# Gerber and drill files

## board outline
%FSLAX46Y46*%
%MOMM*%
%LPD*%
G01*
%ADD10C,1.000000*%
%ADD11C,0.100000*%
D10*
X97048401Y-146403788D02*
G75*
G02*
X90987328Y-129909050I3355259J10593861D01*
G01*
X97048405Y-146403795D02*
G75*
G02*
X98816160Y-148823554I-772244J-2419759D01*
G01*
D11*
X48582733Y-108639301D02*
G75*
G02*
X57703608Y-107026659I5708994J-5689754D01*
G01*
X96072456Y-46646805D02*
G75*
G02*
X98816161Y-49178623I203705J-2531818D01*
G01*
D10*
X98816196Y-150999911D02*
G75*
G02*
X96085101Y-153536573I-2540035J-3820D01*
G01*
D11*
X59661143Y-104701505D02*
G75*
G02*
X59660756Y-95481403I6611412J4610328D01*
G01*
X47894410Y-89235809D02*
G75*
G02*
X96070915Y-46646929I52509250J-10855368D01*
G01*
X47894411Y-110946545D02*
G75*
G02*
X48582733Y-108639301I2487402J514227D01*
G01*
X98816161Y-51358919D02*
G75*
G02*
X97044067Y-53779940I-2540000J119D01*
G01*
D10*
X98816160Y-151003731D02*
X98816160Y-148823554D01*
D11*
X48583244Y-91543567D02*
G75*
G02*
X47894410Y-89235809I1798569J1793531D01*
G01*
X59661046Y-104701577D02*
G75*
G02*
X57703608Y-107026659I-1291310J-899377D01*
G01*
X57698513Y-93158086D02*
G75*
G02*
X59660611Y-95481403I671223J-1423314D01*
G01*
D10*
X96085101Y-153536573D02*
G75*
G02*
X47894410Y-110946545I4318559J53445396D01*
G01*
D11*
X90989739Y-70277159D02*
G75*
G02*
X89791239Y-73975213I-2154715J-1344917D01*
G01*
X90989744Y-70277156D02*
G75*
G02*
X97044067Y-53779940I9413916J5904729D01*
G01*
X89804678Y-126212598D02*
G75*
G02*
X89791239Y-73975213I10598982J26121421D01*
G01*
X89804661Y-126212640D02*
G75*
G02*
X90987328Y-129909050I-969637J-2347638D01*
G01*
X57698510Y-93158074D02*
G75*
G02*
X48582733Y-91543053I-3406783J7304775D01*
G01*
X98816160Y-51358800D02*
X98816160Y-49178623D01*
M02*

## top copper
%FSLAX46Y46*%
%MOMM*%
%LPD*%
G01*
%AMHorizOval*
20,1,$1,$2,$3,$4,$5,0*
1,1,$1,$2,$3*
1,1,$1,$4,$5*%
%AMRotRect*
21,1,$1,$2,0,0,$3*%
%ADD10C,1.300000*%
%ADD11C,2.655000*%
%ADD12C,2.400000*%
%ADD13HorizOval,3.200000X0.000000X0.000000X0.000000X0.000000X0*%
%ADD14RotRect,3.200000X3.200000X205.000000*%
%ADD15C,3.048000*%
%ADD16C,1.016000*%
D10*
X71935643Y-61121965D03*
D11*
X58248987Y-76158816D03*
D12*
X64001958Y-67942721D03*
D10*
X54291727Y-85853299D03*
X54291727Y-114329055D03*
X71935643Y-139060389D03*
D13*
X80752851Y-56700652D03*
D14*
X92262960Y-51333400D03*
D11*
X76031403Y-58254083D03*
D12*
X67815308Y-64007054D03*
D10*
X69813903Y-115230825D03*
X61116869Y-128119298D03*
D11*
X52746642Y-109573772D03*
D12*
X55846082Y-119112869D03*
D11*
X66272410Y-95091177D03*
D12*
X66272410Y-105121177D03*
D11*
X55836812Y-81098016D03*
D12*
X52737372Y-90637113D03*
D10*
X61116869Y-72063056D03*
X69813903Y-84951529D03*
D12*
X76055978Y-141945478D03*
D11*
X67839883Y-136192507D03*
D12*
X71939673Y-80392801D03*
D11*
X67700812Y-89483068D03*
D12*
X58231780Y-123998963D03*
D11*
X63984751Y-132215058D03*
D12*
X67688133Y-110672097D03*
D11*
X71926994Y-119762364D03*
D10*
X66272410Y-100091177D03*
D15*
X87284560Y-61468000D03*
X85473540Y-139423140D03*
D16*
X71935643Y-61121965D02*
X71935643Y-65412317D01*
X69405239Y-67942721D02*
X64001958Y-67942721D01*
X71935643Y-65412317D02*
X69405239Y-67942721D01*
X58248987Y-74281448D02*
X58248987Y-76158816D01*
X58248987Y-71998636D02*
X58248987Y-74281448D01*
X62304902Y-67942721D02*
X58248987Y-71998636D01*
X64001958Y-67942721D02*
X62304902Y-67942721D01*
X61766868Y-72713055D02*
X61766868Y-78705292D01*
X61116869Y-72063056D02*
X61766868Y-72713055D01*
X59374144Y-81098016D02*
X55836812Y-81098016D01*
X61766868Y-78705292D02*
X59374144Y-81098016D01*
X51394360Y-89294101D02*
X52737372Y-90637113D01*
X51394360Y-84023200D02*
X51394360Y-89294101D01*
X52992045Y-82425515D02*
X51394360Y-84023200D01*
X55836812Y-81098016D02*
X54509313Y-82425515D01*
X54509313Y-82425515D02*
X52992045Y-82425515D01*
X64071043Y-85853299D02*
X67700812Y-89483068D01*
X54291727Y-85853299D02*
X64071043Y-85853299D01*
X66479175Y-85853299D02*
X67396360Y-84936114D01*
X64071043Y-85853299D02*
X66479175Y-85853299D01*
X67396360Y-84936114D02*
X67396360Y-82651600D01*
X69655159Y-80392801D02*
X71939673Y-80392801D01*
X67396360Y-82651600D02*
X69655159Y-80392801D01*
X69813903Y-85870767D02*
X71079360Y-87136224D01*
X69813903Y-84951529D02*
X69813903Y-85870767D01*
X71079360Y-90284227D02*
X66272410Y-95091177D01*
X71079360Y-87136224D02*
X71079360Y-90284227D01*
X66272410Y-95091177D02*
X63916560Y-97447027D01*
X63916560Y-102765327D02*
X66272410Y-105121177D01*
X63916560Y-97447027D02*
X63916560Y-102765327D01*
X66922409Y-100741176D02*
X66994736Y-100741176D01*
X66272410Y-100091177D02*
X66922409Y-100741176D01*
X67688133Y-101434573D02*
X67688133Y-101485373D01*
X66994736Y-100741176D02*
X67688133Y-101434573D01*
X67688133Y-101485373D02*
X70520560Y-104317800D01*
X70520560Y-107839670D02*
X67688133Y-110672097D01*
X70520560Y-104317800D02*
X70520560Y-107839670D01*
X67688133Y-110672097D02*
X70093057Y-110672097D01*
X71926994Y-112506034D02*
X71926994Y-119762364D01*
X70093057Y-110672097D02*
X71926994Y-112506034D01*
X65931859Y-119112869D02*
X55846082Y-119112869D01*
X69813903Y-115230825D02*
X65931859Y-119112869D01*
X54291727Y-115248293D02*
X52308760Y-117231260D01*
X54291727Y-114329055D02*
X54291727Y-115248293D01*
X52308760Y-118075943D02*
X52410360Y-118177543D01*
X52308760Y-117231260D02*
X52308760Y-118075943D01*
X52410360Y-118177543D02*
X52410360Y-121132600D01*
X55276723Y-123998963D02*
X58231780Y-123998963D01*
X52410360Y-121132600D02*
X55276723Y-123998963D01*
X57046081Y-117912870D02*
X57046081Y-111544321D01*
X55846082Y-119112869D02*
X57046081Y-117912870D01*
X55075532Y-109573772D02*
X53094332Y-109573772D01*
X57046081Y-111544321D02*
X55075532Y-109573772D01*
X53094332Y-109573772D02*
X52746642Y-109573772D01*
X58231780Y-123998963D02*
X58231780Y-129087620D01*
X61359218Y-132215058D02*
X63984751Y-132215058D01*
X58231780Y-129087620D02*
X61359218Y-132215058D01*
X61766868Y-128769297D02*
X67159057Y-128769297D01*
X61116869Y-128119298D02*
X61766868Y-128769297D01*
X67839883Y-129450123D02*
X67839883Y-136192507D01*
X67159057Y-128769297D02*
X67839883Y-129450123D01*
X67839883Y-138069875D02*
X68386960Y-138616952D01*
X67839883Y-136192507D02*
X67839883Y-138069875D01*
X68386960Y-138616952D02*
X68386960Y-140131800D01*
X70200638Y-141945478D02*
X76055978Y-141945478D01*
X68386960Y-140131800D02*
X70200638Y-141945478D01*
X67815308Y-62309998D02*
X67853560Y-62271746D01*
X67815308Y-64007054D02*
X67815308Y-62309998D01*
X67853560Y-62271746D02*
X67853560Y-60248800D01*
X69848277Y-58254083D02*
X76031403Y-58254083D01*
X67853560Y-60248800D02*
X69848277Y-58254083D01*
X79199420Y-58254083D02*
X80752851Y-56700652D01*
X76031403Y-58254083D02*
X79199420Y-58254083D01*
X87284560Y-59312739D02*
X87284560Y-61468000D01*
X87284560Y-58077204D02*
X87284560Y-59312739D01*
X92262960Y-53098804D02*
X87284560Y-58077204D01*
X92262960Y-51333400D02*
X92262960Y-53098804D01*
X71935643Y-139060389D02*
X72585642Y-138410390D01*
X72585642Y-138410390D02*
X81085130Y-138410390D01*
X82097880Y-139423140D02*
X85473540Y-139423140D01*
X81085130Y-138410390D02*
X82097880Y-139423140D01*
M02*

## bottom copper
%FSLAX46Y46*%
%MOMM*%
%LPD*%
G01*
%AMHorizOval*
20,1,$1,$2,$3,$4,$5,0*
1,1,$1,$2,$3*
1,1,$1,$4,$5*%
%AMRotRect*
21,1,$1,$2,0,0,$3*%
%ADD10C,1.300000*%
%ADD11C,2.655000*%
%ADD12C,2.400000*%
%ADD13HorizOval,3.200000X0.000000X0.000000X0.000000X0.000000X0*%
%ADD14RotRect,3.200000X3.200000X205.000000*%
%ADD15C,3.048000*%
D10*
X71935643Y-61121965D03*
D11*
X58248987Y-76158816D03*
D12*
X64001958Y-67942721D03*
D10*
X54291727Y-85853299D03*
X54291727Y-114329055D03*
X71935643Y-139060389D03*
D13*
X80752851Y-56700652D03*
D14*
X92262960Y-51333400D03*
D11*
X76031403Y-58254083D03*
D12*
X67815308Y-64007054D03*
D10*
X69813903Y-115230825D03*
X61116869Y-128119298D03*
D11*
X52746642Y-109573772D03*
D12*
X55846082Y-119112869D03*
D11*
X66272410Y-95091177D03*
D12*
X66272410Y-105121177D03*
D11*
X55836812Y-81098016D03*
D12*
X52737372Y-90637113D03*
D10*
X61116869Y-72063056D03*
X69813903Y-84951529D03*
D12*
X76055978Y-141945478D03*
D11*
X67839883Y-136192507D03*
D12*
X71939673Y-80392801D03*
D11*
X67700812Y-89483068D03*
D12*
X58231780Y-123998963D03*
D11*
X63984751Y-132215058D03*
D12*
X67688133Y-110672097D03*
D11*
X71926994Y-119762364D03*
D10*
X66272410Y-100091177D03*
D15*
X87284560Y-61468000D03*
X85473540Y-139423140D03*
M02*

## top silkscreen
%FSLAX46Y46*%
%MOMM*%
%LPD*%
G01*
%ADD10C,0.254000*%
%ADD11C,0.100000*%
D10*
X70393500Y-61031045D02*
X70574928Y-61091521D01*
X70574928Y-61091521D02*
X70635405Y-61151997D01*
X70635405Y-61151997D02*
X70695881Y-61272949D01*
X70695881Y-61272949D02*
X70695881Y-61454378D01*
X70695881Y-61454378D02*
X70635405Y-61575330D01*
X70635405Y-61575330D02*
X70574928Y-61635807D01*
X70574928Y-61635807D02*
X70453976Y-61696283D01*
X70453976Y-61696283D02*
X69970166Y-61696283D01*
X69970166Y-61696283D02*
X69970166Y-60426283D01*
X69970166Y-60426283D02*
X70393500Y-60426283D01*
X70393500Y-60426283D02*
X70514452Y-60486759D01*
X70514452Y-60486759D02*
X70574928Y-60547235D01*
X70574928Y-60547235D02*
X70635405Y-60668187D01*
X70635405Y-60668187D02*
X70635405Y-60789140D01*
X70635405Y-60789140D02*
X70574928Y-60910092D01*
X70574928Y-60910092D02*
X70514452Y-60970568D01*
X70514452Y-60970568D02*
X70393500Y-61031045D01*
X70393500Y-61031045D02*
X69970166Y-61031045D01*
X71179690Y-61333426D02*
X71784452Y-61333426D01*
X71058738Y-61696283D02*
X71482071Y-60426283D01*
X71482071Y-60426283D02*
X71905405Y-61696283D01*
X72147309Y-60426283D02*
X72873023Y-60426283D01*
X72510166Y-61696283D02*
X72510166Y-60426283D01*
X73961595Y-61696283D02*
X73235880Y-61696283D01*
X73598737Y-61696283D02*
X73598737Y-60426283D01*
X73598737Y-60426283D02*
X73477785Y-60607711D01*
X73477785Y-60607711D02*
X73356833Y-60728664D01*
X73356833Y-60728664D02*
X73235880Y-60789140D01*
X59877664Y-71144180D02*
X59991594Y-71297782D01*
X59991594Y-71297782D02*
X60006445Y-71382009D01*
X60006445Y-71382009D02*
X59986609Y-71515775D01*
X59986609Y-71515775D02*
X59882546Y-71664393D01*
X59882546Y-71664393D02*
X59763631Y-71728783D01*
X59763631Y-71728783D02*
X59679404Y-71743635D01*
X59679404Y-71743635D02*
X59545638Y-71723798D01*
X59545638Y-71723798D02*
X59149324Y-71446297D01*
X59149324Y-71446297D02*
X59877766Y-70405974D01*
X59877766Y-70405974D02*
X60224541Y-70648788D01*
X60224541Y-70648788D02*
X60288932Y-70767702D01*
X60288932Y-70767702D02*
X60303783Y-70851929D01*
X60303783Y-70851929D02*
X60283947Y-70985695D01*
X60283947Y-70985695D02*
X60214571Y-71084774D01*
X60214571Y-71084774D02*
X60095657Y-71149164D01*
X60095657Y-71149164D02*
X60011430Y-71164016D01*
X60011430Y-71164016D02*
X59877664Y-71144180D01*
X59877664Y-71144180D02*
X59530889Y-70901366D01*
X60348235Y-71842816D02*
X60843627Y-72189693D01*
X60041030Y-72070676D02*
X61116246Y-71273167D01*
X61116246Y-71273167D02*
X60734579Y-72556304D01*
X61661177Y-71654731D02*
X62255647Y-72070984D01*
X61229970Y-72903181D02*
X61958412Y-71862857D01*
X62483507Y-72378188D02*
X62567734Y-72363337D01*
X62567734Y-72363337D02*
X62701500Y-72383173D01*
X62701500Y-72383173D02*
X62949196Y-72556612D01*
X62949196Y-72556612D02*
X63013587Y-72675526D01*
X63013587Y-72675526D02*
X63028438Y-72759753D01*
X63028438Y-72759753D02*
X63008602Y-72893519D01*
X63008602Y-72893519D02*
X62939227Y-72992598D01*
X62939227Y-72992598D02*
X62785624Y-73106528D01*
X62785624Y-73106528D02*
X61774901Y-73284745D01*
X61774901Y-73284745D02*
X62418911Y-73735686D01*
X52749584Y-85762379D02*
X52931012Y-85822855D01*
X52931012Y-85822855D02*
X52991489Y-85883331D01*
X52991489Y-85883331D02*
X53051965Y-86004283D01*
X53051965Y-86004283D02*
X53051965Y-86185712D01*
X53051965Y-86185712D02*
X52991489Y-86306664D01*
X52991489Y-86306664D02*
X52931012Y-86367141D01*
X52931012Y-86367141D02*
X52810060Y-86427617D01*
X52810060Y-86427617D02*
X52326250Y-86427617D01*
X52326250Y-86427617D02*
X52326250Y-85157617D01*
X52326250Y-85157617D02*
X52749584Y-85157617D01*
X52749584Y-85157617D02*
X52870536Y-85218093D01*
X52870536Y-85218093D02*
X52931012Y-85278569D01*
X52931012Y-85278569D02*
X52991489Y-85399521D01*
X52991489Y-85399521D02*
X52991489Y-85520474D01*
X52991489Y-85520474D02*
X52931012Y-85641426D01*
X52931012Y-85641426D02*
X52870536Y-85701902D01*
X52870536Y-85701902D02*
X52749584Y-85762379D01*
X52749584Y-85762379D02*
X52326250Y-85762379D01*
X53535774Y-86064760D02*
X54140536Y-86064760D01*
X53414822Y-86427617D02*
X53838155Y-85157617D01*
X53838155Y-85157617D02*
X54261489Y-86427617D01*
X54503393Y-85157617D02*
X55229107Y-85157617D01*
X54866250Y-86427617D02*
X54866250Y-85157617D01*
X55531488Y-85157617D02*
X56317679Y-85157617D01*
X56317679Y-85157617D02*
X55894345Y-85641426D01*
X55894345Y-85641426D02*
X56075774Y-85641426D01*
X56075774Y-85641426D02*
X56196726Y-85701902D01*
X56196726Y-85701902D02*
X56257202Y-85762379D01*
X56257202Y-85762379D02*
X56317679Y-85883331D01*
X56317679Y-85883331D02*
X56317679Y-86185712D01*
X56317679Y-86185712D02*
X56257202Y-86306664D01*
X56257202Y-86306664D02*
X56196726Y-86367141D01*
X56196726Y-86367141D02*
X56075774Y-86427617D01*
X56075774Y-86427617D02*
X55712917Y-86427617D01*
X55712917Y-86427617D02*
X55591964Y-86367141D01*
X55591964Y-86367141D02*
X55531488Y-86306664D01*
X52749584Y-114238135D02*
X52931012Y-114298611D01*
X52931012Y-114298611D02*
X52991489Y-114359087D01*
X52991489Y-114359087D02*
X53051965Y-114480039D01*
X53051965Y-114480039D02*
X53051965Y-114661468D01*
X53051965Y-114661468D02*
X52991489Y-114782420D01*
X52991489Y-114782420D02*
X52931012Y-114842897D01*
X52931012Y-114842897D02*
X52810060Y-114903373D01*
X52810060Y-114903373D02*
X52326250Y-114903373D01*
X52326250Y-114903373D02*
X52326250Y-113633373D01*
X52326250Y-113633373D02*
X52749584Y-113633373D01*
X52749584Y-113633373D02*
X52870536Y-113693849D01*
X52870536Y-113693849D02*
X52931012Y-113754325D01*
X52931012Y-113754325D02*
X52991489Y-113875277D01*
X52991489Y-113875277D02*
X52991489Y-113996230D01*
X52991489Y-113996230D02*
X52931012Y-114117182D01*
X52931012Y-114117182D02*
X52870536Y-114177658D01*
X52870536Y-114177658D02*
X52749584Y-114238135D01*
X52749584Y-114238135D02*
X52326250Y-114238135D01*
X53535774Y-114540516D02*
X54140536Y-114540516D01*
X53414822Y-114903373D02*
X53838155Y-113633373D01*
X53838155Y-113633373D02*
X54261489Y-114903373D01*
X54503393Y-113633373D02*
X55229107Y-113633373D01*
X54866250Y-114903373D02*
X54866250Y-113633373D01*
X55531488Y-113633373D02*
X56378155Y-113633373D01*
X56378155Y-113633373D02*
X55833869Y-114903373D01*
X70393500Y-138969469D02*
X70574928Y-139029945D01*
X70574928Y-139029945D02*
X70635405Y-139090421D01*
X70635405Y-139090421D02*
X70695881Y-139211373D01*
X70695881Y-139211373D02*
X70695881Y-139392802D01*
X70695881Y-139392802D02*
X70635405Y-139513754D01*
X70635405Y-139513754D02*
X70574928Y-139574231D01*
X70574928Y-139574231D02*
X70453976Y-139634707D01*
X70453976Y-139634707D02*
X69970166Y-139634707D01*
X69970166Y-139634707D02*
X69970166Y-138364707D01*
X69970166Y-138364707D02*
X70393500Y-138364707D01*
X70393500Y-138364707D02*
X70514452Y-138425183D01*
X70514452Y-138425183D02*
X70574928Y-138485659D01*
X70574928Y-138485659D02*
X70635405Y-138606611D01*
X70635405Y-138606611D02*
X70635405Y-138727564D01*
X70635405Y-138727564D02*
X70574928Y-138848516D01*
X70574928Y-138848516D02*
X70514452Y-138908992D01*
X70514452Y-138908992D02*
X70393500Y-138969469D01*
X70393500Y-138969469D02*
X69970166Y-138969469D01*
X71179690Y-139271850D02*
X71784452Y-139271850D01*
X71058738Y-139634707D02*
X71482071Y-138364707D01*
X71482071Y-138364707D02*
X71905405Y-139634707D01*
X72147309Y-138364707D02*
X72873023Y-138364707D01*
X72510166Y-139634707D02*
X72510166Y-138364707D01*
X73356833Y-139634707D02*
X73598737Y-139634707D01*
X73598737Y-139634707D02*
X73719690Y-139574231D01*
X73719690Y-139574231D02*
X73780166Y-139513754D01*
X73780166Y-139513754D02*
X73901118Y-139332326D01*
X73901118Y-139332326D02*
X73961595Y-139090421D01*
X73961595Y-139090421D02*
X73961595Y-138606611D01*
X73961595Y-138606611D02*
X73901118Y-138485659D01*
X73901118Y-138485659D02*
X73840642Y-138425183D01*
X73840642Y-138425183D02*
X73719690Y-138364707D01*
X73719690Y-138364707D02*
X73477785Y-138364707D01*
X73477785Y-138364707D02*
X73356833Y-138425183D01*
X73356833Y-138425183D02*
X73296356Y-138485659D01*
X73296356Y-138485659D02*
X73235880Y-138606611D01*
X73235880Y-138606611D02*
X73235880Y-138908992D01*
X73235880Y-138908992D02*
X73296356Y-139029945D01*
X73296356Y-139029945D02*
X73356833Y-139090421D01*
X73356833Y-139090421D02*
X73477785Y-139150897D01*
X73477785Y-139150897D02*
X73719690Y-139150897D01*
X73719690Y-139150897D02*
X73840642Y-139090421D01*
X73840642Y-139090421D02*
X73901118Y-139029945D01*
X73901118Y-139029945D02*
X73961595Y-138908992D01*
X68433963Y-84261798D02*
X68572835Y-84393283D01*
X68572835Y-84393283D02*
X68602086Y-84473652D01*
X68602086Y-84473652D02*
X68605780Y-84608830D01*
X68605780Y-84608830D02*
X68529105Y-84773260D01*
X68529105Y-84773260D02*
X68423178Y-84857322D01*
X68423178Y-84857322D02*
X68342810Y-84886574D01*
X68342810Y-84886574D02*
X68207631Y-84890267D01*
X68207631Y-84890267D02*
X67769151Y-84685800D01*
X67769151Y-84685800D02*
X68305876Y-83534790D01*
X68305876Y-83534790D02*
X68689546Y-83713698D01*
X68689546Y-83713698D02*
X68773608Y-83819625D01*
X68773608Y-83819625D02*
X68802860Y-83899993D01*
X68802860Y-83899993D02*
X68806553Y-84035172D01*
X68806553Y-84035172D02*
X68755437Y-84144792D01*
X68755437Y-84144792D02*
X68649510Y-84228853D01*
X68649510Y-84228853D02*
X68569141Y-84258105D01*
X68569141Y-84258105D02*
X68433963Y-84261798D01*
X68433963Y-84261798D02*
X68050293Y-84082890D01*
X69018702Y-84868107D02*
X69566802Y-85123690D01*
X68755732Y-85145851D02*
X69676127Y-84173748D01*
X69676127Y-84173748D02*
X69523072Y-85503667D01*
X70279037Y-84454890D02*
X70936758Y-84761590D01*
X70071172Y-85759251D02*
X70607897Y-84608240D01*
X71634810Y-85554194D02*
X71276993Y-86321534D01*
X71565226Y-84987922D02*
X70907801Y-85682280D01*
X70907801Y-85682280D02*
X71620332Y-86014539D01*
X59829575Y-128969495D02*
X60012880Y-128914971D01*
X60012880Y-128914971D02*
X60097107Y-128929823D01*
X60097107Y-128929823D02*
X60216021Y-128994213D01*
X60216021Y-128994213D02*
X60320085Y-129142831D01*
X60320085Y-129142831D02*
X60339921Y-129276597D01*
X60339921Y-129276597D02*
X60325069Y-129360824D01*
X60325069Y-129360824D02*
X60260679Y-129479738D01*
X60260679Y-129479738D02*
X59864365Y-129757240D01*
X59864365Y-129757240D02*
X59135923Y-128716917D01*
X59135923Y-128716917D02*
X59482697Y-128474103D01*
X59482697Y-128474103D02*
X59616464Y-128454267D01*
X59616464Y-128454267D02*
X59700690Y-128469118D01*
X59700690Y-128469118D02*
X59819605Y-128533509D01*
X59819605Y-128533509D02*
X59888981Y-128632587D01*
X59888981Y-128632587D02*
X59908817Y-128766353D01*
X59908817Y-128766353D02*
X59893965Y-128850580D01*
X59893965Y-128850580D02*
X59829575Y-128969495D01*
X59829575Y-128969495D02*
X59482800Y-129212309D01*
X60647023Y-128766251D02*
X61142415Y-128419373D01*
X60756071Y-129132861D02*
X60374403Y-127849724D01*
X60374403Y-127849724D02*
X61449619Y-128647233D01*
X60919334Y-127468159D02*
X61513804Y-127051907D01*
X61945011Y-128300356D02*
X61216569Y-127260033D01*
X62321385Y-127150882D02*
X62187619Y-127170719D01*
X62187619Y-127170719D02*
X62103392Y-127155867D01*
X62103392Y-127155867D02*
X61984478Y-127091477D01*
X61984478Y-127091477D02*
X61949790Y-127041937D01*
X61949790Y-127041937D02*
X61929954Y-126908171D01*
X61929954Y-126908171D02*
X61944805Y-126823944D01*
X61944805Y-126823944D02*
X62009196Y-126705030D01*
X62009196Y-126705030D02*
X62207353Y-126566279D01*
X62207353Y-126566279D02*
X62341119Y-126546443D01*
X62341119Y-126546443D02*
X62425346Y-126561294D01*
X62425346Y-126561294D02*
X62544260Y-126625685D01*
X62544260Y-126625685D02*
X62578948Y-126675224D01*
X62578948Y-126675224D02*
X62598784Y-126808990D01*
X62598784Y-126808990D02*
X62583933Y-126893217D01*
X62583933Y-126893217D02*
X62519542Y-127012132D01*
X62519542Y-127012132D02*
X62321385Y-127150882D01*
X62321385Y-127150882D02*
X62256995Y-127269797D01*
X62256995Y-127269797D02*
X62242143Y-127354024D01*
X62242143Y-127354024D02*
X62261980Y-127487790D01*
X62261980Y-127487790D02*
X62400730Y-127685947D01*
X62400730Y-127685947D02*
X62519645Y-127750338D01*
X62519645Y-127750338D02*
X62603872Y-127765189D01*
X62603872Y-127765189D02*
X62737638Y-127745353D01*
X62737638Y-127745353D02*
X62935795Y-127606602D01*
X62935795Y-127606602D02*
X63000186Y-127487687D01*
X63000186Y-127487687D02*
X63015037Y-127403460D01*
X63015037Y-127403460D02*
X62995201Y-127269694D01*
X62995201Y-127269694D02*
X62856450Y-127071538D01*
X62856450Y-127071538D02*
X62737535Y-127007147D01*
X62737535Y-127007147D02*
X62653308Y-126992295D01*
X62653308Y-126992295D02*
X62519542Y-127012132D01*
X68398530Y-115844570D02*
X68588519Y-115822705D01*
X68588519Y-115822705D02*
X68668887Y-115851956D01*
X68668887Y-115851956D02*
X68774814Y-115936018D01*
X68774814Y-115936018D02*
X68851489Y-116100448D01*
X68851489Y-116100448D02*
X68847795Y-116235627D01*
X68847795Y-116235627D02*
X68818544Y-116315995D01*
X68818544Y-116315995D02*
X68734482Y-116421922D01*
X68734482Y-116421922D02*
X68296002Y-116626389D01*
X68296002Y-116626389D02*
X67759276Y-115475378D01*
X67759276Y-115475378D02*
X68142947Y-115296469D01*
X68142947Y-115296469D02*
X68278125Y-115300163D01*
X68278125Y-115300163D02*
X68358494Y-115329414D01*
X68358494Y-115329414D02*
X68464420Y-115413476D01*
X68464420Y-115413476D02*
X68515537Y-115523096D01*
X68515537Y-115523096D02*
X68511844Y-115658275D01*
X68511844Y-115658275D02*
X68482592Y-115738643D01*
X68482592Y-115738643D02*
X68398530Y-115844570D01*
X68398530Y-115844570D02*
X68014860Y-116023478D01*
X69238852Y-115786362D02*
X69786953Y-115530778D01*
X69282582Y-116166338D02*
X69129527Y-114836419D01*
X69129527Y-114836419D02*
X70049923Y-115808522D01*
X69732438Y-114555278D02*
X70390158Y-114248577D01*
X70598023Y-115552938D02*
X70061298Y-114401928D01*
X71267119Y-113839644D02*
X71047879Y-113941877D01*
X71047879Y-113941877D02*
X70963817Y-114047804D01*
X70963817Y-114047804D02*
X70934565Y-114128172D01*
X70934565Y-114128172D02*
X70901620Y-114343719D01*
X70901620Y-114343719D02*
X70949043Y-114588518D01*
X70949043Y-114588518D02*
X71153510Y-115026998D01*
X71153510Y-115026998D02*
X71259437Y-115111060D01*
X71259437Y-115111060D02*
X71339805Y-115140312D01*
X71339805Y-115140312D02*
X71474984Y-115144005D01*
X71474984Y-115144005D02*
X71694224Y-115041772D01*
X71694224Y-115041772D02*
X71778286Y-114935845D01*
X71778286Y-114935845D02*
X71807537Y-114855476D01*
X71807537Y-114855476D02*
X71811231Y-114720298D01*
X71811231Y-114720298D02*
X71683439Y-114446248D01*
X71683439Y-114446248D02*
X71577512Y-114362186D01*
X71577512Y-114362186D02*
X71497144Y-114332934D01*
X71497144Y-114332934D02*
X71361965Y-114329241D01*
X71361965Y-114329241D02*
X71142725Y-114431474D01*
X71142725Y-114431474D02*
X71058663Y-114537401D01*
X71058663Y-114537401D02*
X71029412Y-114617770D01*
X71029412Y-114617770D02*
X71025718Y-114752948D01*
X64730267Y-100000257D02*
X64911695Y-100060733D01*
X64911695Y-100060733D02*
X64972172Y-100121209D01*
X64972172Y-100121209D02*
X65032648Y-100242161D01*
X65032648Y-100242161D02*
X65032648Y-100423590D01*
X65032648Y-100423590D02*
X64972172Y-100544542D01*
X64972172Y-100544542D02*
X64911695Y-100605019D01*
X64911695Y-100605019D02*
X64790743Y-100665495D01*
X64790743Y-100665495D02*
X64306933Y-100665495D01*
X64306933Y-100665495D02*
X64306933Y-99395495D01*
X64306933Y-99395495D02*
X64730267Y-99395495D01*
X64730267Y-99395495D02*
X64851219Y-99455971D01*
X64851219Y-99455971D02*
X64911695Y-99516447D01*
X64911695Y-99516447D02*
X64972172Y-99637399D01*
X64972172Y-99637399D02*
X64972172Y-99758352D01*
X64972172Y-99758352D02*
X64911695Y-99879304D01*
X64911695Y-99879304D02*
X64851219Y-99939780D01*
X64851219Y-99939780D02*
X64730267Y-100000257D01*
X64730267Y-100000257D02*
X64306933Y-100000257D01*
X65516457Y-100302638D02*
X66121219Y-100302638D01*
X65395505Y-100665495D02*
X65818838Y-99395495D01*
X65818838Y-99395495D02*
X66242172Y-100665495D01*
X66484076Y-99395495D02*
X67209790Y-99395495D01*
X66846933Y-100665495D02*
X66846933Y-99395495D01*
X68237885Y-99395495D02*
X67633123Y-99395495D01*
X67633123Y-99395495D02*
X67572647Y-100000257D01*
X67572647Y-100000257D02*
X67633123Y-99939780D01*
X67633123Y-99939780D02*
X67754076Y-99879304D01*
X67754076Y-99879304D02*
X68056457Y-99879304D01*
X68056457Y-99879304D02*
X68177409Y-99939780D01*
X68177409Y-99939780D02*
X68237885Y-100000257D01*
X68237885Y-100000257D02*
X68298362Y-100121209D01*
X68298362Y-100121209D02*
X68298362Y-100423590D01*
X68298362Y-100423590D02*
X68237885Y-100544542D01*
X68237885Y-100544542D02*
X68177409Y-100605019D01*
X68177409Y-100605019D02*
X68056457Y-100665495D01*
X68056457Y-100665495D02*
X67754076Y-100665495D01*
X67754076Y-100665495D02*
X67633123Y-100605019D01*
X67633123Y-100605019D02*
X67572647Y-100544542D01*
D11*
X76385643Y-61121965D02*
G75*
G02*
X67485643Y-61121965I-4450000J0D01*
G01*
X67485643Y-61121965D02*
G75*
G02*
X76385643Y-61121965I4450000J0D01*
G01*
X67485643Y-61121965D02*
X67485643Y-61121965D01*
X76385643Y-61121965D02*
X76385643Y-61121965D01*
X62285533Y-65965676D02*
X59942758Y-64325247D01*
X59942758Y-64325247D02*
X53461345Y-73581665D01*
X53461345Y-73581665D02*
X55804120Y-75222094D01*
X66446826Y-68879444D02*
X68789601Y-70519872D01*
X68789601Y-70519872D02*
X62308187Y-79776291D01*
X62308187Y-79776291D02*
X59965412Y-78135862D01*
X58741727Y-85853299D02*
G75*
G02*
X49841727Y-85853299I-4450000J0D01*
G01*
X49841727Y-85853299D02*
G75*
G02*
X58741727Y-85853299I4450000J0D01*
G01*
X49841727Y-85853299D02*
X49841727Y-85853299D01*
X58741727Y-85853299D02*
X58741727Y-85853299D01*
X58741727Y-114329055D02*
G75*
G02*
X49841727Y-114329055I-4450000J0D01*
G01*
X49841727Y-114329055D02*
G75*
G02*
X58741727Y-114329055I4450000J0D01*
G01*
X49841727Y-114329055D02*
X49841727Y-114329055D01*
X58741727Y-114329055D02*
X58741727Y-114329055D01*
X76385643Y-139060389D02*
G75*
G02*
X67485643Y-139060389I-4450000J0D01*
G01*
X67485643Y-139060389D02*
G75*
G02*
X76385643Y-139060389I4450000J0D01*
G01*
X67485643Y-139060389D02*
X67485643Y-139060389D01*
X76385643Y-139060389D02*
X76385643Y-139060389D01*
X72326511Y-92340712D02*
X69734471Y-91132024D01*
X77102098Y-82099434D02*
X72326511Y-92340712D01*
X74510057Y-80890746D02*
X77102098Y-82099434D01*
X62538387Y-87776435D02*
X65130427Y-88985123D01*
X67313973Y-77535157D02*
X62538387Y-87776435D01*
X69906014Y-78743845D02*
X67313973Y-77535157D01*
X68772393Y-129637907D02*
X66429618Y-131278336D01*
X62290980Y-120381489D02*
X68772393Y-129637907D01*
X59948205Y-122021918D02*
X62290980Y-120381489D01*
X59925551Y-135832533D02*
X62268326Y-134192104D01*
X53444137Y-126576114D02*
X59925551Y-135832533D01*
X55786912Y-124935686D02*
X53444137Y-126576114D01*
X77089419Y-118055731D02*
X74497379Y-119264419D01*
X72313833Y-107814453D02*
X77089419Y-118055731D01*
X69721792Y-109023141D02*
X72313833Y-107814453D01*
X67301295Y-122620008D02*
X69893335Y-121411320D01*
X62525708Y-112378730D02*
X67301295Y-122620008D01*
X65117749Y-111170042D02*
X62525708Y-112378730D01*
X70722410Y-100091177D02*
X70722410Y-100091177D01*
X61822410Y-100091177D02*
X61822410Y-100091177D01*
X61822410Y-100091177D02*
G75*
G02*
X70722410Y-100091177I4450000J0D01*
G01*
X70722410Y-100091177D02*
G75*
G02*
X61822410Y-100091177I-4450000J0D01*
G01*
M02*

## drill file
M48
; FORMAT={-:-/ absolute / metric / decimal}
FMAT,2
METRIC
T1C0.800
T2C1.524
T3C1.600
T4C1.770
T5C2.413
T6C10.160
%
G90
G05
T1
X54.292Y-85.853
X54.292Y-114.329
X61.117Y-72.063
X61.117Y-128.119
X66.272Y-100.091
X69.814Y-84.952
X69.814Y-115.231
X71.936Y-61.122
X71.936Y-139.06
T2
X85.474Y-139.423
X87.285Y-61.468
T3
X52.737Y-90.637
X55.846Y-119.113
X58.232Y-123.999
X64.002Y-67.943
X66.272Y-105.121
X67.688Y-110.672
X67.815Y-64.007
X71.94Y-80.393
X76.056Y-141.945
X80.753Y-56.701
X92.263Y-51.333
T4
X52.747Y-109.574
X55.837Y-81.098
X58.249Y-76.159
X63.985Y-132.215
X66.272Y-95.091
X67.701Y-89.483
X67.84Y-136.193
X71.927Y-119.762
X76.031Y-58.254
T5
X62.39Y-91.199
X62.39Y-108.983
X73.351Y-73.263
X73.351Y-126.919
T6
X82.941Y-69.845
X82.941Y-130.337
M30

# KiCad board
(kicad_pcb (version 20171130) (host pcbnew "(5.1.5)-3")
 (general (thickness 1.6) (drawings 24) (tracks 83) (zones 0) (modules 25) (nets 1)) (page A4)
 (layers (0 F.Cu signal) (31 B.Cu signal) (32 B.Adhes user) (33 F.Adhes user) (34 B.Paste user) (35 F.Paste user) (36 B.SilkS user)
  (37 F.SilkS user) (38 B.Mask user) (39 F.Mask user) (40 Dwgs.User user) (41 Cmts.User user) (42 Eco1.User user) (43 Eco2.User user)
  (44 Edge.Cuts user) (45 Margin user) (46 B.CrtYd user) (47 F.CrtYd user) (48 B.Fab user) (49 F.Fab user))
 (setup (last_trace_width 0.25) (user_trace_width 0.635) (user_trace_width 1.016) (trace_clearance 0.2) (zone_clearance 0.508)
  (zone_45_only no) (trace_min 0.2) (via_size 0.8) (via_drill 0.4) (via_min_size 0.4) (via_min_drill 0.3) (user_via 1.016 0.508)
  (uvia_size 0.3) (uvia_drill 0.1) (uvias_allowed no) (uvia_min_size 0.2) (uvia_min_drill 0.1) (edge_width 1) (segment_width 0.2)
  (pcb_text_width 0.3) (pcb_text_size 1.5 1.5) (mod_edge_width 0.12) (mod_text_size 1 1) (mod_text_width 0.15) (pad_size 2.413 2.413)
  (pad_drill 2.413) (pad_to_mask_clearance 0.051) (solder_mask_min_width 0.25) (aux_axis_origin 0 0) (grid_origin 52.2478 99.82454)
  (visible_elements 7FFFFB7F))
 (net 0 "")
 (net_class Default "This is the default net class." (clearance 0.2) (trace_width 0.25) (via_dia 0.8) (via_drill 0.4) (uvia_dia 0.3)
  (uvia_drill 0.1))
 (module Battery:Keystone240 (layer F.Cu) (at 71.935643 61.121965 180)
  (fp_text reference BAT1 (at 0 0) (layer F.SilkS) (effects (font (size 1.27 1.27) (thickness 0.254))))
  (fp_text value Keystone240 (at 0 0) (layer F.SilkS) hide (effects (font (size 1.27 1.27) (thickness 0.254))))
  (fp_arc (start 0 0) (end 4.45 0) (angle -180) (layer F.SilkS) (width 0.1))
  (fp_arc (start 0 0) (end -4.45 0) (angle -180) (layer F.SilkS) (width 0.1))
  (fp_line (start 4.45 0) (end 4.45 0) (layer F.SilkS) (width 0.1))
  (fp_line (start -4.45 0) (end -4.45 0) (layer F.SilkS) (width 0.1))
  (pad 1 thru_hole circle (at 0 0 180) (size 1.3 1.3) (drill 0.8) (layers *.Cu *.Mask)))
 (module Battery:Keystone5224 (layer F.Cu) (at 61.116869 72.063056 325)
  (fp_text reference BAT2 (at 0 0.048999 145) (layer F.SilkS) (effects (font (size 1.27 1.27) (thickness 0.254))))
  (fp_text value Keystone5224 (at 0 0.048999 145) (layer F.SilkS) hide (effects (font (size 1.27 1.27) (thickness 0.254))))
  (fp_line (start -2.54 -5.665) (end -5.4 -5.665) (layer F.SilkS) (width 0.1))
  (fp_line (start -5.4 -5.665) (end -5.4 5.635) (layer F.SilkS) (width 0.1))
  (fp_line (start -5.4 5.635) (end -2.54 5.635) (layer F.SilkS) (width 0.1))
  (fp_line (start 2.54 -5.665) (end 5.4 -5.665) (layer F.SilkS) (width 0.1))
  (fp_line (start 5.4 -5.665) (end 5.4 5.635) (layer F.SilkS) (width 0.1))
  (fp_line (start 5.4 5.635) (end 2.54 5.635) (layer F.SilkS) (width 0.1))
  (pad 1 thru_hole circle (at 0 5 325) (size 2.655 2.655) (drill 1.77) (layers *.Cu *.Mask))
  (pad 2 thru_hole circle (at 0 -5.03 325) (size 2.4 2.4) (drill 1.6) (layers *.Cu *.Mask)))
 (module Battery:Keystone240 (layer F.Cu) (at 54.291727 85.853299 180)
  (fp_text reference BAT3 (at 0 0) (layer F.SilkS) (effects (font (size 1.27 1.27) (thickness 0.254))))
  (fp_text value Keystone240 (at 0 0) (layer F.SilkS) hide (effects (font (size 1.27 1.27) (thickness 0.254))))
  (fp_arc (start 0 0) (end 4.45 0) (angle -180) (layer F.SilkS) (width 0.1))
  (fp_arc (start 0 0) (end -4.45 0) (angle -180) (layer F.SilkS) (width 0.1))
  (fp_line (start 4.45 0) (end 4.45 0) (layer F.SilkS) (width 0.1))
  (fp_line (start -4.45 0) (end -4.45 0) (layer F.SilkS) (width 0.1))
  (pad 1 thru_hole circle (at 0 0 180) (size 1.3 1.3) (drill 0.8) (layers *.Cu *.Mask)))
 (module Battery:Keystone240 (layer F.Cu) (at 54.291727 114.329055 180)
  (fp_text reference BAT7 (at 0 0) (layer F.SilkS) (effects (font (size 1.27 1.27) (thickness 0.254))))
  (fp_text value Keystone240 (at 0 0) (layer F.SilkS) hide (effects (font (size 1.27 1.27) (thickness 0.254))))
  (fp_arc (start 0 0) (end 4.45 0) (angle -180) (layer F.SilkS) (width 0.1))
  (fp_arc (start 0 0) (end -4.45 0) (angle -180) (layer F.SilkS) (width 0.1))
  (fp_line (start 4.45 0) (end 4.45 0) (layer F.SilkS) (width 0.1))
  (fp_line (start -4.45 0) (end -4.45 0) (layer F.SilkS) (width 0.1))
  (pad 1 thru_hole circle (at 0 0 180) (size 1.3 1.3) (drill 0.8) (layers *.Cu *.Mask)))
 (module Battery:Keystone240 (layer F.Cu) (at 71.935643 139.060389 180)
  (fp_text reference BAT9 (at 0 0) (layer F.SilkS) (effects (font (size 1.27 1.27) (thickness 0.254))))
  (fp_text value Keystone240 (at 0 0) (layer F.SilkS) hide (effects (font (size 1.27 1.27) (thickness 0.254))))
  (fp_arc (start 0 0) (end 4.45 0) (angle -180) (layer F.SilkS) (width 0.1))
  (fp_arc (start 0 0) (end -4.45 0) (angle -180) (layer F.SilkS) (width 0.1))
  (fp_line (start 4.45 0) (end 4.45 0) (layer F.SilkS) (width 0.1))
  (fp_line (start -4.45 0) (end -4.45 0) (layer F.SilkS) (width 0.1))
  (pad 1 thru_hole circle (at 0 0 180) (size 1.3 1.3) (drill 0.8) (layers *.Cu *.Mask)))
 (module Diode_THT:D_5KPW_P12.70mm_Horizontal (layer B.Cu) (at 92.26296 51.3334 205)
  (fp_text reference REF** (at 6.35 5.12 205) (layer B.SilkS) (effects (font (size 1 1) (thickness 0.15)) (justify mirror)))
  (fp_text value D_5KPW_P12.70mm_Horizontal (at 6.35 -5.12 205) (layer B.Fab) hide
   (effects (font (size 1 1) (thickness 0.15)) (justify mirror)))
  (pad 2 thru_hole oval (at 12.7 0 205) (size 3.2 3.2) (drill 1.6) (layers *.Cu *.Mask))
  (pad 1 thru_hole rect (at 0 0 205) (size 3.2 3.2) (drill 1.6) (layers *.Cu *.Mask)))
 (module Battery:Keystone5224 (layer B.Cu) (at 71.935643 61.121965 305)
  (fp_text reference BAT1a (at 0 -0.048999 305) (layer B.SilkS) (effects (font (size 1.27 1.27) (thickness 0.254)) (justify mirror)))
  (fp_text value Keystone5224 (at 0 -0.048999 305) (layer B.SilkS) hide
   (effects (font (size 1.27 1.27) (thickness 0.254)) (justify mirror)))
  (pad 1 thru_hole circle (at 0 -5 305) (size 2.655 2.655) (drill 1.77) (layers *.Cu *.Mask))
  (pad 2 thru_hole circle (at 0 5.03 305) (size 2.4 2.4) (drill 1.6) (layers *.Cu *.Mask)))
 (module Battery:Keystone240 (layer B.Cu) (at 69.813903 115.230825 180)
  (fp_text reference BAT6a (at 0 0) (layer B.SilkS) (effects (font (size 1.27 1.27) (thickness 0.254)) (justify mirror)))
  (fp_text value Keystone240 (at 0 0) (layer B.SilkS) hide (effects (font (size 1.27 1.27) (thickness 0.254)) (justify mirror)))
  (pad 1 thru_hole circle (at 0 0 180) (size 1.3 1.3) (drill 0.8) (layers *.Cu *.Mask)))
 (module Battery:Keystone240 (layer B.Cu) (at 61.116869 128.119298 180)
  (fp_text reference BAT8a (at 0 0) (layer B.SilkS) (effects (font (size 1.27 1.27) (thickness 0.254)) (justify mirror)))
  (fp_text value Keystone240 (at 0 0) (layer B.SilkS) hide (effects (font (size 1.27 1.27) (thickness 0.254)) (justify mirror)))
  (pad 1 thru_hole circle (at 0 0 180) (size 1.3 1.3) (drill 0.8) (layers *.Cu *.Mask)))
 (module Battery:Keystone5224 (layer B.Cu) (at 54.291727 114.329055 18)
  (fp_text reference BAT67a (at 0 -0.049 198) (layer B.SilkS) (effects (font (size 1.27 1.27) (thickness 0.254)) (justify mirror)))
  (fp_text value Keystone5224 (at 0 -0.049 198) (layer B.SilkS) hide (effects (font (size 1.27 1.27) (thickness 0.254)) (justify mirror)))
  (pad 1 thru_hole circle (at 0 -5 18) (size 2.655 2.655) (drill 1.77) (layers *.Cu *.Mask))
  (pad 2 thru_hole circle (at 0 5.03 18) (size 2.4 2.4) (drill 1.6) (layers *.Cu *.Mask)))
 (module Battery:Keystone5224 (layer B.Cu) (at 66.27241 100.091177)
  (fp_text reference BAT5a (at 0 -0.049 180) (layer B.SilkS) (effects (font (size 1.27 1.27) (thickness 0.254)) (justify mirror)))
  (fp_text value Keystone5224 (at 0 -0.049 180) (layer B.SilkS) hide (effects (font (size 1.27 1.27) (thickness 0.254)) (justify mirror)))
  (pad 1 thru_hole circle (at 0 -5) (size 2.655 2.655) (drill 1.77) (layers *.Cu *.Mask))
  (pad 2 thru_hole circle (at 0 5.03) (size 2.4 2.4) (drill 1.6) (layers *.Cu *.Mask)))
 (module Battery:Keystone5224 (layer B.Cu) (at 54.291727 85.853299 342)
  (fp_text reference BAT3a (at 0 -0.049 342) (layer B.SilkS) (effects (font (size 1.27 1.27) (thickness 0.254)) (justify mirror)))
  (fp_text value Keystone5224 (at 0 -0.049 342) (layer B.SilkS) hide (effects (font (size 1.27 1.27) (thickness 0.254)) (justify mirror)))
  (pad 1 thru_hole circle (at 0 -5 342) (size 2.655 2.655) (drill 1.77) (layers *.Cu *.Mask))
  (pad 2 thru_hole circle (at 0 5.03 342) (size 2.4 2.4) (drill 1.6) (layers *.Cu *.Mask)))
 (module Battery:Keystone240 (layer B.Cu) (at 61.116869 72.063056 180)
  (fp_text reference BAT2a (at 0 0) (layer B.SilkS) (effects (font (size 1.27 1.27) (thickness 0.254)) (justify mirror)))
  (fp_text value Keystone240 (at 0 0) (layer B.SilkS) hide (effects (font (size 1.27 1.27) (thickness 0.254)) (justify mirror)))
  (pad 1 thru_hole circle (at 0 0 180) (size 1.3 1.3) (drill 0.8) (layers *.Cu *.Mask)))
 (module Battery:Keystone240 (layer B.Cu) (at 69.813903 84.951529 180)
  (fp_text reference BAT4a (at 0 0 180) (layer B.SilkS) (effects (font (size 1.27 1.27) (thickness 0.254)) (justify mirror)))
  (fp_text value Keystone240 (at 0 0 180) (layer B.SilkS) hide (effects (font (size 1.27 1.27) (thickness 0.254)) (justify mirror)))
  (pad 1 thru_hole circle (at 0 0 180) (size 1.3 1.3) (drill 0.8) (layers *.Cu *.Mask)))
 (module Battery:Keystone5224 (layer B.Cu) (at 71.935643 139.060389 55)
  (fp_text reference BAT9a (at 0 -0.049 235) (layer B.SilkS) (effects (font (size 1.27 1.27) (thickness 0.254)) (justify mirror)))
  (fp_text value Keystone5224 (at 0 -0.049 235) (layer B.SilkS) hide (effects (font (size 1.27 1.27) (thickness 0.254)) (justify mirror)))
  (pad 2 thru_hole circle (at 0 5.03 55) (size 2.4 2.4) (drill 1.6) (layers *.Cu *.Mask))
  (pad 1 thru_hole circle (at 0 -5 55) (size 2.655 2.655) (drill 1.77) (layers *.Cu *.Mask)))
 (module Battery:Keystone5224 (layer F.Cu) (at 69.813903 84.951529 335)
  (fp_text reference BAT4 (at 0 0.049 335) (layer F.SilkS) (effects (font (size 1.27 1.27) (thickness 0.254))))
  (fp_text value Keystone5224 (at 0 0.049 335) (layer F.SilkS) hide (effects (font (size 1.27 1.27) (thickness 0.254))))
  (fp_line (start 5.4 5.635) (end 2.54 5.635) (layer F.SilkS) (width 0.1))
  (fp_line (start 5.4 -5.665) (end 5.4 5.635) (layer F.SilkS) (width 0.1))
  (fp_line (start 2.54 -5.665) (end 5.4 -5.665) (layer F.SilkS) (width 0.1))
  (fp_line (start -5.4 5.635) (end -2.54 5.635) (layer F.SilkS) (width 0.1))
  (fp_line (start -5.4 -5.665) (end -5.4 5.635) (layer F.SilkS) (width 0.1))
  (fp_line (start -2.54 -5.665) (end -5.4 -5.665) (layer F.SilkS) (width 0.1))
  (pad 2 thru_hole circle (at 0 -5.03 335) (size 2.4 2.4) (drill 1.6) (layers *.Cu *.Mask))
  (pad 1 thru_hole circle (at 0 5 335) (size 2.655 2.655) (drill 1.77) (layers *.Cu *.Mask)))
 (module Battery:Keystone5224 (layer F.Cu) (at 61.116869 128.119298 35)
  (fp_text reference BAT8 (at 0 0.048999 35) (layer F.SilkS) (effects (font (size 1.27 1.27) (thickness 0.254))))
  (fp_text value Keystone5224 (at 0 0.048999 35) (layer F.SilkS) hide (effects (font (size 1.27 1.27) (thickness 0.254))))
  (fp_line (start 5.4 5.635) (end 2.54 5.635) (layer F.SilkS) (width 0.1))
  (fp_line (start 5.4 -5.665) (end 5.4 5.635) (layer F.SilkS) (width 0.1))
  (fp_line (start 2.54 -5.665) (end 5.4 -5.665) (layer F.SilkS) (width 0.1))
  (fp_line (start -5.4 5.635) (end -2.54 5.635) (layer F.SilkS) (width 0.1))
  (fp_line (start -5.4 -5.665) (end -5.4 5.635) (layer F.SilkS) (width 0.1))
  (fp_line (start -2.54 -5.665) (end -5.4 -5.665) (layer F.SilkS) (width 0.1))
  (pad 2 thru_hole circle (at 0 -5.03 35) (size 2.4 2.4) (drill 1.6) (layers *.Cu *.Mask))
  (pad 1 thru_hole circle (at 0 5 35) (size 2.655 2.655) (drill 1.77) (layers *.Cu *.Mask)))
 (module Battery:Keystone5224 (layer F.Cu) (at 69.813903 115.230825 25)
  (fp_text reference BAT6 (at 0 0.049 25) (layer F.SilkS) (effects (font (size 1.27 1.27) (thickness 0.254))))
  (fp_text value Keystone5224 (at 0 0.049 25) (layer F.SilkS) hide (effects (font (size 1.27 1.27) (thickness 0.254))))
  (fp_line (start 5.4 5.635) (end 2.54 5.635) (layer F.SilkS) (width 0.1))
  (fp_line (start 5.4 -5.665) (end 5.4 5.635) (layer F.SilkS) (width 0.1))
  (fp_line (start 2.54 -5.665) (end 5.4 -5.665) (layer F.SilkS) (width 0.1))
  (fp_line (start -5.4 5.635) (end -2.54 5.635) (layer F.SilkS) (width 0.1))
  (fp_line (start -5.4 -5.665) (end -5.4 5.635) (layer F.SilkS) (width 0.1))
  (fp_line (start -2.54 -5.665) (end -5.4 -5.665) (layer F.SilkS) (width 0.1))
  (pad 2 thru_hole circle (at 0 -5.03 25) (size 2.4 2.4) (drill 1.6) (layers *.Cu *.Mask))
  (pad 1 thru_hole circle (at 0 5 25) (size 2.655 2.655) (drill 1.77) (layers *.Cu *.Mask)))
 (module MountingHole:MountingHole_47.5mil (layer F.Cu) (at 73.350759 73.263011)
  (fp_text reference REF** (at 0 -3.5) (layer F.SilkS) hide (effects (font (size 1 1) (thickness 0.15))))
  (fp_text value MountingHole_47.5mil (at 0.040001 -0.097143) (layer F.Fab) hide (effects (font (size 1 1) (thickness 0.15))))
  (pad "" np_thru_hole circle (at 0 0) (size 2.413 2.413) (drill 2.413) (layers *.Cu *.Mask)))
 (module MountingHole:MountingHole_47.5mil (layer F.Cu) (at 62.389563 91.198855)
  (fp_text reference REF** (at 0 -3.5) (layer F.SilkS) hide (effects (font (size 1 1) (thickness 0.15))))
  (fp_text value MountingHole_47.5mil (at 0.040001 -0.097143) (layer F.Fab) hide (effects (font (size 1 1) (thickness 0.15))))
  (pad "" np_thru_hole circle (at 0 0) (size 2.413 2.413) (drill 2.413) (layers *.Cu *.Mask)))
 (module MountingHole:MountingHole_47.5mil (layer F.Cu) (at 62.389563 108.983499)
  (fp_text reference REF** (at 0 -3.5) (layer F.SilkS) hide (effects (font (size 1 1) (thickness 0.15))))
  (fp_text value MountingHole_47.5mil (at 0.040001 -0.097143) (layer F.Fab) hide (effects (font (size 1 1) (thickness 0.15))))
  (pad "" np_thru_hole circle (at 0 0) (size 2.413 2.413) (drill 2.413) (layers *.Cu *.Mask)))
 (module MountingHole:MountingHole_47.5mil (layer F.Cu) (at 73.350759 126.919343)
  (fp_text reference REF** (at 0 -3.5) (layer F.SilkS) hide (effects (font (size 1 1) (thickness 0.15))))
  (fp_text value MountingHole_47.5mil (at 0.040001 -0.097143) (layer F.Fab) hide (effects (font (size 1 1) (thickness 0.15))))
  (pad "" np_thru_hole circle (at 0 0) (size 2.413 2.413) (drill 2.413) (layers *.Cu *.Mask)))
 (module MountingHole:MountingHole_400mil (layer F.Cu) (at 82.94116 130.337114)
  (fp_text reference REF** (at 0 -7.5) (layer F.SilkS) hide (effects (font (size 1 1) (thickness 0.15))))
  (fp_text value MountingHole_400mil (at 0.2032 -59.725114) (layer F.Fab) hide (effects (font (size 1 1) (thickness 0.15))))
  (pad "" np_thru_hole circle (at 0 0) (size 10.16 10.16) (drill 10.16) (layers *.Cu *.Mask)))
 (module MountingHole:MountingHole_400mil (layer F.Cu) (at 82.94116 69.84524)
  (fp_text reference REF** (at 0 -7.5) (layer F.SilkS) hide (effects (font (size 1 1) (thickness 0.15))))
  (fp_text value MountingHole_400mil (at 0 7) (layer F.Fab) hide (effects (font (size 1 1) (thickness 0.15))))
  (pad "" np_thru_hole circle (at 0 0) (size 10.16 10.16) (drill 10.16) (layers *.Cu *.Mask)))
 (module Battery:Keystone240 (layer F.Cu) (at 66.27241 100.091177 180)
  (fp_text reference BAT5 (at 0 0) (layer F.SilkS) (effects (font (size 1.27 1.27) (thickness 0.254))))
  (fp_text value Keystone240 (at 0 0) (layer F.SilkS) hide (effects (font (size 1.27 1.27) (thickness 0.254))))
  (fp_line (start -4.45 0) (end -4.45 0) (layer F.SilkS) (width 0.1))
  (fp_line (start 4.45 0) (end 4.45 0) (layer F.SilkS) (width 0.1))
  (fp_arc (start 0 0) (end -4.45 0) (angle -180) (layer F.SilkS) (width 0.1))
  (fp_arc (start 0 0) (end 4.45 0) (angle -180) (layer F.SilkS) (width 0.1))
  (pad 1 thru_hole circle (at 0 0 180) (size 1.3 1.3) (drill 0.8) (layers *.Cu *.Mask)))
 (gr_arc (start 100.40366 135.809927) (end 90.987328 129.90905) (angle -104.5) (layer Edge.Cuts) (width 1))
 (gr_arc (start 96.276161 148.823554) (end 98.81616 148.823554) (angle -72.3) (layer Edge.Cuts) (width 1))
 (gr_arc (start 54.291727 114.329055) (end 57.703608 107.026659) (angle -70.13998941) (layer Edge.Cuts) (width 0.1))
 (gr_arc (start 96.276161 49.178623) (end 98.816161 49.178623) (angle -94.6) (layer Edge.Cuts) (width 0.1))
 (gr_arc (start 96.276161 151.003731) (end 96.085101 153.536573) (angle -94.4) (layer Edge.Cuts) (width 1))
 (gr_arc (start 66.272555 100.091177) (end 59.660756 95.481403) (angle -69.77354428) (layer Edge.Cuts) (width 0.1))
 (gr_arc (start 100.40366 100.091177) (end 96.070915 46.646929) (angle -73.68479152) (layer Edge.Cuts) (width 0.1))
 (gr_arc (start 50.381813 110.432318) (end 48.582733 108.639301) (angle -56.5836465) (layer Edge.Cuts) (width 0.1))
 (gr_arc (start 96.276161 51.3588) (end 97.044067 53.77994) (angle -72.4) (layer Edge.Cuts) (width 0.1))
 (gr_line (start 98.81616 151.003731) (end 98.81616 148.823554) (layer Edge.Cuts) (width 1))
 (gr_arc (start 50.381813 89.750036) (end 47.89441 89.235809) (angle -56.6) (layer Edge.Cuts) (width 0.1))
 (gr_arc (start 58.369736 105.600954) (end 57.703608 107.026659) (angle -149.8998569) (layer Edge.Cuts) (width 0.1))
 (gr_arc (start 58.369736 94.5814) (end 59.660611 95.481403) (angle -150.13253) (layer Edge.Cuts) (width 0.1))
 (gr_arc (start 100.40366 100.091177) (end 47.89441 110.946545) (angle -73.7) (layer Edge.Cuts) (width 1))
 (gr_arc (start 88.835024 71.622076) (end 89.791239 73.975213) (angle -99.85659665) (layer Edge.Cuts) (width 0.1))
 (gr_arc (start 100.40366 64.372427) (end 97.044067 53.77994) (angle -104.5) (layer Edge.Cuts) (width 0.1))
 (gr_arc (start 100.40366 100.091177) (end 89.791239 73.975213) (angle -135.8) (layer Edge.Cuts) (width 0.1))
 (gr_arc (start 88.835024 128.560278) (end 90.987328 129.90905) (angle -99.63198075) (layer Edge.Cuts) (width 0.1))
 (gr_arc (start 54.291727 85.853299) (end 48.582733 91.543053) (angle -70.1) (layer Edge.Cuts) (width 0.1))
 (gr_line (start 98.81616 51.3588) (end 98.81616 49.178623) (layer Edge.Cuts) (width 0.1))
 (segment (start 71.935643 61.121965) (end 71.935643 65.412317) (width 1.016) (layer F.Cu) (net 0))
 (segment (start 69.405239 67.942721) (end 64.001958 67.942721) (width 1.016) (layer F.Cu) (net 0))
 (segment (start 71.935643 65.412317) (end 69.405239 67.942721) (width 1.016) (layer F.Cu) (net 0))
 (segment (start 58.248987 74.281448) (end 58.248987 76.158816) (width 1.016) (layer F.Cu) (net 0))
 (segment (start 58.248987 71.998636) (end 58.248987 74.281448) (width 1.016) (layer F.Cu) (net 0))
 (segment (start 62.304902 67.942721) (end 58.248987 71.998636) (width 1.016) (layer F.Cu) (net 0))
 (segment (start 64.001958 67.942721) (end 62.304902 67.942721) (width 1.016) (layer F.Cu) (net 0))
 (segment (start 61.766868 72.713055) (end 61.766868 78.705292) (width 1.016) (layer F.Cu) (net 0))
 (segment (start 61.116869 72.063056) (end 61.766868 72.713055) (width 1.016) (layer F.Cu) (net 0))
 (segment (start 59.374144 81.098016) (end 55.836812 81.098016) (width 1.016) (layer F.Cu) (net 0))
 (segment (start 61.766868 78.705292) (end 59.374144 81.098016) (width 1.016) (layer F.Cu) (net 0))
 (segment (start 51.39436 89.294101) (end 52.737372 90.637113) (width 1.016) (layer F.Cu) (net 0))
 (segment (start 51.39436 84.0232) (end 51.39436 89.294101) (width 1.016) (layer F.Cu) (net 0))
 (segment (start 52.992045 82.425515) (end 51.39436 84.0232) (width 1.016) (layer F.Cu) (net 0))
 (segment (start 55.836812 81.098016) (end 54.509313 82.425515) (width 1.016) (layer F.Cu) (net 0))
 (segment (start 54.509313 82.425515) (end 52.992045 82.425515) (width 1.016) (layer F.Cu) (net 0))
 (segment (start 64.071043 85.853299) (end 67.700812 89.483068) (width 1.016) (layer F.Cu) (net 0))
 (segment (start 54.291727 85.853299) (end 64.071043 85.853299) (width 1.016) (layer F.Cu) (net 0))
 (segment (start 66.479175 85.853299) (end 67.39636 84.936114) (width 1.016) (layer F.Cu) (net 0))
 (segment (start 64.071043 85.853299) (end 66.479175 85.853299) (width 1.016) (layer F.Cu) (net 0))
 (segment (start 67.39636 84.936114) (end 67.39636 82.6516) (width 1.016) (layer F.Cu) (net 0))
 (segment (start 69.655159 80.392801) (end 71.939673 80.392801) (width 1.016) (layer F.Cu) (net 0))
 (segment (start 67.39636 82.6516) (end 69.655159 80.392801) (width 1.016) (layer F.Cu) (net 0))
 (segment (start 69.813903 85.870767) (end 71.07936 87.136224) (width 1.016) (layer F.Cu) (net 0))
 (segment (start 69.813903 84.951529) (end 69.813903 85.870767) (width 1.016) (layer F.Cu) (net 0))
 (segment (start 71.07936 90.284227) (end 66.27241 95.091177) (width 1.016) (layer F.Cu) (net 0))
 (segment (start 71.07936 87.136224) (end 71.07936 90.284227) (width 1.016) (layer F.Cu) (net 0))
 (segment (start 66.27241 95.091177) (end 63.91656 97.447027) (width 1.016) (layer F.Cu) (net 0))
 (segment (start 63.91656 102.765327) (end 66.27241 105.121177) (width 1.016) (layer F.Cu) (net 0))
 (segment (start 63.91656 97.447027) (end 63.91656 102.765327) (width 1.016) (layer F.Cu) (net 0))
 (segment (start 66.922409 100.741176) (end 66.994736 100.741176) (width 1.016) (layer F.Cu) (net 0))
 (segment (start 66.27241 100.091177) (end 66.922409 100.741176) (width 1.016) (layer F.Cu) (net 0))
 (segment (start 67.688133 101.434573) (end 67.688133 101.485373) (width 1.016) (layer F.Cu) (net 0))
 (segment (start 66.994736 100.741176) (end 67.688133 101.434573) (width 1.016) (layer F.Cu) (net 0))
 (segment (start 67.688133 101.485373) (end 70.52056 104.3178) (width 1.016) (layer F.Cu) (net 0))
 (segment (start 70.52056 107.83967) (end 67.688133 110.672097) (width 1.016) (layer F.Cu) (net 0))
 (segment (start 70.52056 104.3178) (end 70.52056 107.83967) (width 1.016) (layer F.Cu) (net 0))
 (segment (start 67.688133 110.672097) (end 70.093057 110.672097) (width 1.016) (layer F.Cu) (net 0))
 (segment (start 71.926994 112.506034) (end 71.926994 119.762364) (width 1.016) (layer F.Cu) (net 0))
 (segment (start 70.093057 110.672097) (end 71.926994 112.506034) (width 1.016) (layer F.Cu) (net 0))
 (segment (start 65.931859 119.112869) (end 55.846082 119.112869) (width 1.016) (layer F.Cu) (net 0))
 (segment (start 69.813903 115.230825) (end 65.931859 119.112869) (width 1.016) (layer F.Cu) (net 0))
 (segment (start 54.291727 115.248293) (end 52.30876 117.23126) (width 1.016) (layer F.Cu) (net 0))
 (segment (start 54.291727 114.329055) (end 54.291727 115.248293) (width 1.016) (layer F.Cu) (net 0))
 (segment (start 52.30876 118.075943) (end 52.41036 118.177543) (width 1.016) (layer F.Cu) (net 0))
 (segment (start 52.30876 117.23126) (end 52.30876 118.075943) (width 1.016) (layer F.Cu) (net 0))
 (segment (start 52.41036 118.177543) (end 52.41036 121.1326) (width 1.016) (layer F.Cu) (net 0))
 (segment (start 55.276723 123.998963) (end 58.23178 123.998963) (width 1.016) (layer F.Cu) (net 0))
 (segment (start 52.41036 121.1326) (end 55.276723 123.998963) (width 1.016) (layer F.Cu) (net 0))
 (segment (start 57.046081 117.91287) (end 57.046081 111.544321) (width 1.016) (layer F.Cu) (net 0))
 (segment (start 55.846082 119.112869) (end 57.046081 117.91287) (width 1.016) (layer F.Cu) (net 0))
 (segment (start 55.075532 109.573772) (end 53.094332 109.573772) (width 1.016) (layer F.Cu) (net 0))
 (segment (start 57.046081 111.544321) (end 55.075532 109.573772) (width 1.016) (layer F.Cu) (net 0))
 (segment (start 53.094332 109.573772) (end 52.746642 109.573772) (width 1.016) (layer F.Cu) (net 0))
 (segment (start 58.23178 123.998963) (end 58.23178 129.08762) (width 1.016) (layer F.Cu) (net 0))
 (segment (start 61.359218 132.215058) (end 63.984751 132.215058) (width 1.016) (layer F.Cu) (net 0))
 (segment (start 58.23178 129.08762) (end 61.359218 132.215058) (width 1.016) (layer F.Cu) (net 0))
 (segment (start 61.766868 128.769297) (end 67.159057 128.769297) (width 1.016) (layer F.Cu) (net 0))
 (segment (start 61.116869 128.119298) (end 61.766868 128.769297) (width 1.016) (layer F.Cu) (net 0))
 (segment (start 67.839883 129.450123) (end 67.839883 136.192507) (width 1.016) (layer F.Cu) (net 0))
 (segment (start 67.159057 128.769297) (end 67.839883 129.450123) (width 1.016) (layer F.Cu) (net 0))
 (segment (start 67.839883 138.069875) (end 68.38696 138.616952) (width 1.016) (layer F.Cu) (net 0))
 (segment (start 67.839883 136.192507) (end 67.839883 138.069875) (width 1.016) (layer F.Cu) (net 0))
 (segment (start 68.38696 138.616952) (end 68.38696 140.1318) (width 1.016) (layer F.Cu) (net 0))
 (segment (start 70.200638 141.945478) (end 76.055978 141.945478) (width 1.016) (layer F.Cu) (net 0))
 (segment (start 68.38696 140.1318) (end 70.200638 141.945478) (width 1.016) (layer F.Cu) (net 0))
 (segment (start 67.815308 62.309998) (end 67.85356 62.271746) (width 1.016) (layer F.Cu) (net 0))
 (segment (start 67.815308 64.007054) (end 67.815308 62.309998) (width 1.016) (layer F.Cu) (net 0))
 (segment (start 67.85356 62.271746) (end 67.85356 60.2488) (width 1.016) (layer F.Cu) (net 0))
 (segment (start 69.848277 58.254083) (end 76.031403 58.254083) (width 1.016) (layer F.Cu) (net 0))
 (segment (start 67.85356 60.2488) (end 69.848277 58.254083) (width 1.016) (layer F.Cu) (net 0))
 (segment (start 79.19942 58.254083) (end 80.752851 56.700652) (width 1.016) (layer F.Cu) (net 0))
 (segment (start 76.031403 58.254083) (end 79.19942 58.254083) (width 1.016) (layer F.Cu) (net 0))
 (via (at 87.28456 61.468) (size 3.048) (drill 1.524) (layers F.Cu B.Cu) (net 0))
 (segment (start 87.28456 59.312739) (end 87.28456 61.468) (width 1.016) (layer F.Cu) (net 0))
 (segment (start 87.28456 58.077204) (end 87.28456 59.312739) (width 1.016) (layer F.Cu) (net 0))
 (segment (start 92.26296 53.098804) (end 87.28456 58.077204) (width 1.016) (layer F.Cu) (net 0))
 (segment (start 92.26296 51.3334) (end 92.26296 53.098804) (width 1.016) (layer F.Cu) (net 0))
 (via (at 85.47354 139.42314) (size 3.048) (drill 1.524) (layers F.Cu B.Cu) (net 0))
 (segment (start 71.935643 139.060389) (end 72.585642 138.41039) (width 1.016) (layer F.Cu) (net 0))
 (segment (start 72.585642 138.41039) (end 81.08513 138.41039) (width 1.016) (layer F.Cu) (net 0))
 (segment (start 82.09788 139.42314) (end 85.47354 139.42314) (width 1.016) (layer F.Cu) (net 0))
 (segment (start 81.08513 138.41039) (end 82.09788 139.42314) (width 1.016) (layer F.Cu) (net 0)))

